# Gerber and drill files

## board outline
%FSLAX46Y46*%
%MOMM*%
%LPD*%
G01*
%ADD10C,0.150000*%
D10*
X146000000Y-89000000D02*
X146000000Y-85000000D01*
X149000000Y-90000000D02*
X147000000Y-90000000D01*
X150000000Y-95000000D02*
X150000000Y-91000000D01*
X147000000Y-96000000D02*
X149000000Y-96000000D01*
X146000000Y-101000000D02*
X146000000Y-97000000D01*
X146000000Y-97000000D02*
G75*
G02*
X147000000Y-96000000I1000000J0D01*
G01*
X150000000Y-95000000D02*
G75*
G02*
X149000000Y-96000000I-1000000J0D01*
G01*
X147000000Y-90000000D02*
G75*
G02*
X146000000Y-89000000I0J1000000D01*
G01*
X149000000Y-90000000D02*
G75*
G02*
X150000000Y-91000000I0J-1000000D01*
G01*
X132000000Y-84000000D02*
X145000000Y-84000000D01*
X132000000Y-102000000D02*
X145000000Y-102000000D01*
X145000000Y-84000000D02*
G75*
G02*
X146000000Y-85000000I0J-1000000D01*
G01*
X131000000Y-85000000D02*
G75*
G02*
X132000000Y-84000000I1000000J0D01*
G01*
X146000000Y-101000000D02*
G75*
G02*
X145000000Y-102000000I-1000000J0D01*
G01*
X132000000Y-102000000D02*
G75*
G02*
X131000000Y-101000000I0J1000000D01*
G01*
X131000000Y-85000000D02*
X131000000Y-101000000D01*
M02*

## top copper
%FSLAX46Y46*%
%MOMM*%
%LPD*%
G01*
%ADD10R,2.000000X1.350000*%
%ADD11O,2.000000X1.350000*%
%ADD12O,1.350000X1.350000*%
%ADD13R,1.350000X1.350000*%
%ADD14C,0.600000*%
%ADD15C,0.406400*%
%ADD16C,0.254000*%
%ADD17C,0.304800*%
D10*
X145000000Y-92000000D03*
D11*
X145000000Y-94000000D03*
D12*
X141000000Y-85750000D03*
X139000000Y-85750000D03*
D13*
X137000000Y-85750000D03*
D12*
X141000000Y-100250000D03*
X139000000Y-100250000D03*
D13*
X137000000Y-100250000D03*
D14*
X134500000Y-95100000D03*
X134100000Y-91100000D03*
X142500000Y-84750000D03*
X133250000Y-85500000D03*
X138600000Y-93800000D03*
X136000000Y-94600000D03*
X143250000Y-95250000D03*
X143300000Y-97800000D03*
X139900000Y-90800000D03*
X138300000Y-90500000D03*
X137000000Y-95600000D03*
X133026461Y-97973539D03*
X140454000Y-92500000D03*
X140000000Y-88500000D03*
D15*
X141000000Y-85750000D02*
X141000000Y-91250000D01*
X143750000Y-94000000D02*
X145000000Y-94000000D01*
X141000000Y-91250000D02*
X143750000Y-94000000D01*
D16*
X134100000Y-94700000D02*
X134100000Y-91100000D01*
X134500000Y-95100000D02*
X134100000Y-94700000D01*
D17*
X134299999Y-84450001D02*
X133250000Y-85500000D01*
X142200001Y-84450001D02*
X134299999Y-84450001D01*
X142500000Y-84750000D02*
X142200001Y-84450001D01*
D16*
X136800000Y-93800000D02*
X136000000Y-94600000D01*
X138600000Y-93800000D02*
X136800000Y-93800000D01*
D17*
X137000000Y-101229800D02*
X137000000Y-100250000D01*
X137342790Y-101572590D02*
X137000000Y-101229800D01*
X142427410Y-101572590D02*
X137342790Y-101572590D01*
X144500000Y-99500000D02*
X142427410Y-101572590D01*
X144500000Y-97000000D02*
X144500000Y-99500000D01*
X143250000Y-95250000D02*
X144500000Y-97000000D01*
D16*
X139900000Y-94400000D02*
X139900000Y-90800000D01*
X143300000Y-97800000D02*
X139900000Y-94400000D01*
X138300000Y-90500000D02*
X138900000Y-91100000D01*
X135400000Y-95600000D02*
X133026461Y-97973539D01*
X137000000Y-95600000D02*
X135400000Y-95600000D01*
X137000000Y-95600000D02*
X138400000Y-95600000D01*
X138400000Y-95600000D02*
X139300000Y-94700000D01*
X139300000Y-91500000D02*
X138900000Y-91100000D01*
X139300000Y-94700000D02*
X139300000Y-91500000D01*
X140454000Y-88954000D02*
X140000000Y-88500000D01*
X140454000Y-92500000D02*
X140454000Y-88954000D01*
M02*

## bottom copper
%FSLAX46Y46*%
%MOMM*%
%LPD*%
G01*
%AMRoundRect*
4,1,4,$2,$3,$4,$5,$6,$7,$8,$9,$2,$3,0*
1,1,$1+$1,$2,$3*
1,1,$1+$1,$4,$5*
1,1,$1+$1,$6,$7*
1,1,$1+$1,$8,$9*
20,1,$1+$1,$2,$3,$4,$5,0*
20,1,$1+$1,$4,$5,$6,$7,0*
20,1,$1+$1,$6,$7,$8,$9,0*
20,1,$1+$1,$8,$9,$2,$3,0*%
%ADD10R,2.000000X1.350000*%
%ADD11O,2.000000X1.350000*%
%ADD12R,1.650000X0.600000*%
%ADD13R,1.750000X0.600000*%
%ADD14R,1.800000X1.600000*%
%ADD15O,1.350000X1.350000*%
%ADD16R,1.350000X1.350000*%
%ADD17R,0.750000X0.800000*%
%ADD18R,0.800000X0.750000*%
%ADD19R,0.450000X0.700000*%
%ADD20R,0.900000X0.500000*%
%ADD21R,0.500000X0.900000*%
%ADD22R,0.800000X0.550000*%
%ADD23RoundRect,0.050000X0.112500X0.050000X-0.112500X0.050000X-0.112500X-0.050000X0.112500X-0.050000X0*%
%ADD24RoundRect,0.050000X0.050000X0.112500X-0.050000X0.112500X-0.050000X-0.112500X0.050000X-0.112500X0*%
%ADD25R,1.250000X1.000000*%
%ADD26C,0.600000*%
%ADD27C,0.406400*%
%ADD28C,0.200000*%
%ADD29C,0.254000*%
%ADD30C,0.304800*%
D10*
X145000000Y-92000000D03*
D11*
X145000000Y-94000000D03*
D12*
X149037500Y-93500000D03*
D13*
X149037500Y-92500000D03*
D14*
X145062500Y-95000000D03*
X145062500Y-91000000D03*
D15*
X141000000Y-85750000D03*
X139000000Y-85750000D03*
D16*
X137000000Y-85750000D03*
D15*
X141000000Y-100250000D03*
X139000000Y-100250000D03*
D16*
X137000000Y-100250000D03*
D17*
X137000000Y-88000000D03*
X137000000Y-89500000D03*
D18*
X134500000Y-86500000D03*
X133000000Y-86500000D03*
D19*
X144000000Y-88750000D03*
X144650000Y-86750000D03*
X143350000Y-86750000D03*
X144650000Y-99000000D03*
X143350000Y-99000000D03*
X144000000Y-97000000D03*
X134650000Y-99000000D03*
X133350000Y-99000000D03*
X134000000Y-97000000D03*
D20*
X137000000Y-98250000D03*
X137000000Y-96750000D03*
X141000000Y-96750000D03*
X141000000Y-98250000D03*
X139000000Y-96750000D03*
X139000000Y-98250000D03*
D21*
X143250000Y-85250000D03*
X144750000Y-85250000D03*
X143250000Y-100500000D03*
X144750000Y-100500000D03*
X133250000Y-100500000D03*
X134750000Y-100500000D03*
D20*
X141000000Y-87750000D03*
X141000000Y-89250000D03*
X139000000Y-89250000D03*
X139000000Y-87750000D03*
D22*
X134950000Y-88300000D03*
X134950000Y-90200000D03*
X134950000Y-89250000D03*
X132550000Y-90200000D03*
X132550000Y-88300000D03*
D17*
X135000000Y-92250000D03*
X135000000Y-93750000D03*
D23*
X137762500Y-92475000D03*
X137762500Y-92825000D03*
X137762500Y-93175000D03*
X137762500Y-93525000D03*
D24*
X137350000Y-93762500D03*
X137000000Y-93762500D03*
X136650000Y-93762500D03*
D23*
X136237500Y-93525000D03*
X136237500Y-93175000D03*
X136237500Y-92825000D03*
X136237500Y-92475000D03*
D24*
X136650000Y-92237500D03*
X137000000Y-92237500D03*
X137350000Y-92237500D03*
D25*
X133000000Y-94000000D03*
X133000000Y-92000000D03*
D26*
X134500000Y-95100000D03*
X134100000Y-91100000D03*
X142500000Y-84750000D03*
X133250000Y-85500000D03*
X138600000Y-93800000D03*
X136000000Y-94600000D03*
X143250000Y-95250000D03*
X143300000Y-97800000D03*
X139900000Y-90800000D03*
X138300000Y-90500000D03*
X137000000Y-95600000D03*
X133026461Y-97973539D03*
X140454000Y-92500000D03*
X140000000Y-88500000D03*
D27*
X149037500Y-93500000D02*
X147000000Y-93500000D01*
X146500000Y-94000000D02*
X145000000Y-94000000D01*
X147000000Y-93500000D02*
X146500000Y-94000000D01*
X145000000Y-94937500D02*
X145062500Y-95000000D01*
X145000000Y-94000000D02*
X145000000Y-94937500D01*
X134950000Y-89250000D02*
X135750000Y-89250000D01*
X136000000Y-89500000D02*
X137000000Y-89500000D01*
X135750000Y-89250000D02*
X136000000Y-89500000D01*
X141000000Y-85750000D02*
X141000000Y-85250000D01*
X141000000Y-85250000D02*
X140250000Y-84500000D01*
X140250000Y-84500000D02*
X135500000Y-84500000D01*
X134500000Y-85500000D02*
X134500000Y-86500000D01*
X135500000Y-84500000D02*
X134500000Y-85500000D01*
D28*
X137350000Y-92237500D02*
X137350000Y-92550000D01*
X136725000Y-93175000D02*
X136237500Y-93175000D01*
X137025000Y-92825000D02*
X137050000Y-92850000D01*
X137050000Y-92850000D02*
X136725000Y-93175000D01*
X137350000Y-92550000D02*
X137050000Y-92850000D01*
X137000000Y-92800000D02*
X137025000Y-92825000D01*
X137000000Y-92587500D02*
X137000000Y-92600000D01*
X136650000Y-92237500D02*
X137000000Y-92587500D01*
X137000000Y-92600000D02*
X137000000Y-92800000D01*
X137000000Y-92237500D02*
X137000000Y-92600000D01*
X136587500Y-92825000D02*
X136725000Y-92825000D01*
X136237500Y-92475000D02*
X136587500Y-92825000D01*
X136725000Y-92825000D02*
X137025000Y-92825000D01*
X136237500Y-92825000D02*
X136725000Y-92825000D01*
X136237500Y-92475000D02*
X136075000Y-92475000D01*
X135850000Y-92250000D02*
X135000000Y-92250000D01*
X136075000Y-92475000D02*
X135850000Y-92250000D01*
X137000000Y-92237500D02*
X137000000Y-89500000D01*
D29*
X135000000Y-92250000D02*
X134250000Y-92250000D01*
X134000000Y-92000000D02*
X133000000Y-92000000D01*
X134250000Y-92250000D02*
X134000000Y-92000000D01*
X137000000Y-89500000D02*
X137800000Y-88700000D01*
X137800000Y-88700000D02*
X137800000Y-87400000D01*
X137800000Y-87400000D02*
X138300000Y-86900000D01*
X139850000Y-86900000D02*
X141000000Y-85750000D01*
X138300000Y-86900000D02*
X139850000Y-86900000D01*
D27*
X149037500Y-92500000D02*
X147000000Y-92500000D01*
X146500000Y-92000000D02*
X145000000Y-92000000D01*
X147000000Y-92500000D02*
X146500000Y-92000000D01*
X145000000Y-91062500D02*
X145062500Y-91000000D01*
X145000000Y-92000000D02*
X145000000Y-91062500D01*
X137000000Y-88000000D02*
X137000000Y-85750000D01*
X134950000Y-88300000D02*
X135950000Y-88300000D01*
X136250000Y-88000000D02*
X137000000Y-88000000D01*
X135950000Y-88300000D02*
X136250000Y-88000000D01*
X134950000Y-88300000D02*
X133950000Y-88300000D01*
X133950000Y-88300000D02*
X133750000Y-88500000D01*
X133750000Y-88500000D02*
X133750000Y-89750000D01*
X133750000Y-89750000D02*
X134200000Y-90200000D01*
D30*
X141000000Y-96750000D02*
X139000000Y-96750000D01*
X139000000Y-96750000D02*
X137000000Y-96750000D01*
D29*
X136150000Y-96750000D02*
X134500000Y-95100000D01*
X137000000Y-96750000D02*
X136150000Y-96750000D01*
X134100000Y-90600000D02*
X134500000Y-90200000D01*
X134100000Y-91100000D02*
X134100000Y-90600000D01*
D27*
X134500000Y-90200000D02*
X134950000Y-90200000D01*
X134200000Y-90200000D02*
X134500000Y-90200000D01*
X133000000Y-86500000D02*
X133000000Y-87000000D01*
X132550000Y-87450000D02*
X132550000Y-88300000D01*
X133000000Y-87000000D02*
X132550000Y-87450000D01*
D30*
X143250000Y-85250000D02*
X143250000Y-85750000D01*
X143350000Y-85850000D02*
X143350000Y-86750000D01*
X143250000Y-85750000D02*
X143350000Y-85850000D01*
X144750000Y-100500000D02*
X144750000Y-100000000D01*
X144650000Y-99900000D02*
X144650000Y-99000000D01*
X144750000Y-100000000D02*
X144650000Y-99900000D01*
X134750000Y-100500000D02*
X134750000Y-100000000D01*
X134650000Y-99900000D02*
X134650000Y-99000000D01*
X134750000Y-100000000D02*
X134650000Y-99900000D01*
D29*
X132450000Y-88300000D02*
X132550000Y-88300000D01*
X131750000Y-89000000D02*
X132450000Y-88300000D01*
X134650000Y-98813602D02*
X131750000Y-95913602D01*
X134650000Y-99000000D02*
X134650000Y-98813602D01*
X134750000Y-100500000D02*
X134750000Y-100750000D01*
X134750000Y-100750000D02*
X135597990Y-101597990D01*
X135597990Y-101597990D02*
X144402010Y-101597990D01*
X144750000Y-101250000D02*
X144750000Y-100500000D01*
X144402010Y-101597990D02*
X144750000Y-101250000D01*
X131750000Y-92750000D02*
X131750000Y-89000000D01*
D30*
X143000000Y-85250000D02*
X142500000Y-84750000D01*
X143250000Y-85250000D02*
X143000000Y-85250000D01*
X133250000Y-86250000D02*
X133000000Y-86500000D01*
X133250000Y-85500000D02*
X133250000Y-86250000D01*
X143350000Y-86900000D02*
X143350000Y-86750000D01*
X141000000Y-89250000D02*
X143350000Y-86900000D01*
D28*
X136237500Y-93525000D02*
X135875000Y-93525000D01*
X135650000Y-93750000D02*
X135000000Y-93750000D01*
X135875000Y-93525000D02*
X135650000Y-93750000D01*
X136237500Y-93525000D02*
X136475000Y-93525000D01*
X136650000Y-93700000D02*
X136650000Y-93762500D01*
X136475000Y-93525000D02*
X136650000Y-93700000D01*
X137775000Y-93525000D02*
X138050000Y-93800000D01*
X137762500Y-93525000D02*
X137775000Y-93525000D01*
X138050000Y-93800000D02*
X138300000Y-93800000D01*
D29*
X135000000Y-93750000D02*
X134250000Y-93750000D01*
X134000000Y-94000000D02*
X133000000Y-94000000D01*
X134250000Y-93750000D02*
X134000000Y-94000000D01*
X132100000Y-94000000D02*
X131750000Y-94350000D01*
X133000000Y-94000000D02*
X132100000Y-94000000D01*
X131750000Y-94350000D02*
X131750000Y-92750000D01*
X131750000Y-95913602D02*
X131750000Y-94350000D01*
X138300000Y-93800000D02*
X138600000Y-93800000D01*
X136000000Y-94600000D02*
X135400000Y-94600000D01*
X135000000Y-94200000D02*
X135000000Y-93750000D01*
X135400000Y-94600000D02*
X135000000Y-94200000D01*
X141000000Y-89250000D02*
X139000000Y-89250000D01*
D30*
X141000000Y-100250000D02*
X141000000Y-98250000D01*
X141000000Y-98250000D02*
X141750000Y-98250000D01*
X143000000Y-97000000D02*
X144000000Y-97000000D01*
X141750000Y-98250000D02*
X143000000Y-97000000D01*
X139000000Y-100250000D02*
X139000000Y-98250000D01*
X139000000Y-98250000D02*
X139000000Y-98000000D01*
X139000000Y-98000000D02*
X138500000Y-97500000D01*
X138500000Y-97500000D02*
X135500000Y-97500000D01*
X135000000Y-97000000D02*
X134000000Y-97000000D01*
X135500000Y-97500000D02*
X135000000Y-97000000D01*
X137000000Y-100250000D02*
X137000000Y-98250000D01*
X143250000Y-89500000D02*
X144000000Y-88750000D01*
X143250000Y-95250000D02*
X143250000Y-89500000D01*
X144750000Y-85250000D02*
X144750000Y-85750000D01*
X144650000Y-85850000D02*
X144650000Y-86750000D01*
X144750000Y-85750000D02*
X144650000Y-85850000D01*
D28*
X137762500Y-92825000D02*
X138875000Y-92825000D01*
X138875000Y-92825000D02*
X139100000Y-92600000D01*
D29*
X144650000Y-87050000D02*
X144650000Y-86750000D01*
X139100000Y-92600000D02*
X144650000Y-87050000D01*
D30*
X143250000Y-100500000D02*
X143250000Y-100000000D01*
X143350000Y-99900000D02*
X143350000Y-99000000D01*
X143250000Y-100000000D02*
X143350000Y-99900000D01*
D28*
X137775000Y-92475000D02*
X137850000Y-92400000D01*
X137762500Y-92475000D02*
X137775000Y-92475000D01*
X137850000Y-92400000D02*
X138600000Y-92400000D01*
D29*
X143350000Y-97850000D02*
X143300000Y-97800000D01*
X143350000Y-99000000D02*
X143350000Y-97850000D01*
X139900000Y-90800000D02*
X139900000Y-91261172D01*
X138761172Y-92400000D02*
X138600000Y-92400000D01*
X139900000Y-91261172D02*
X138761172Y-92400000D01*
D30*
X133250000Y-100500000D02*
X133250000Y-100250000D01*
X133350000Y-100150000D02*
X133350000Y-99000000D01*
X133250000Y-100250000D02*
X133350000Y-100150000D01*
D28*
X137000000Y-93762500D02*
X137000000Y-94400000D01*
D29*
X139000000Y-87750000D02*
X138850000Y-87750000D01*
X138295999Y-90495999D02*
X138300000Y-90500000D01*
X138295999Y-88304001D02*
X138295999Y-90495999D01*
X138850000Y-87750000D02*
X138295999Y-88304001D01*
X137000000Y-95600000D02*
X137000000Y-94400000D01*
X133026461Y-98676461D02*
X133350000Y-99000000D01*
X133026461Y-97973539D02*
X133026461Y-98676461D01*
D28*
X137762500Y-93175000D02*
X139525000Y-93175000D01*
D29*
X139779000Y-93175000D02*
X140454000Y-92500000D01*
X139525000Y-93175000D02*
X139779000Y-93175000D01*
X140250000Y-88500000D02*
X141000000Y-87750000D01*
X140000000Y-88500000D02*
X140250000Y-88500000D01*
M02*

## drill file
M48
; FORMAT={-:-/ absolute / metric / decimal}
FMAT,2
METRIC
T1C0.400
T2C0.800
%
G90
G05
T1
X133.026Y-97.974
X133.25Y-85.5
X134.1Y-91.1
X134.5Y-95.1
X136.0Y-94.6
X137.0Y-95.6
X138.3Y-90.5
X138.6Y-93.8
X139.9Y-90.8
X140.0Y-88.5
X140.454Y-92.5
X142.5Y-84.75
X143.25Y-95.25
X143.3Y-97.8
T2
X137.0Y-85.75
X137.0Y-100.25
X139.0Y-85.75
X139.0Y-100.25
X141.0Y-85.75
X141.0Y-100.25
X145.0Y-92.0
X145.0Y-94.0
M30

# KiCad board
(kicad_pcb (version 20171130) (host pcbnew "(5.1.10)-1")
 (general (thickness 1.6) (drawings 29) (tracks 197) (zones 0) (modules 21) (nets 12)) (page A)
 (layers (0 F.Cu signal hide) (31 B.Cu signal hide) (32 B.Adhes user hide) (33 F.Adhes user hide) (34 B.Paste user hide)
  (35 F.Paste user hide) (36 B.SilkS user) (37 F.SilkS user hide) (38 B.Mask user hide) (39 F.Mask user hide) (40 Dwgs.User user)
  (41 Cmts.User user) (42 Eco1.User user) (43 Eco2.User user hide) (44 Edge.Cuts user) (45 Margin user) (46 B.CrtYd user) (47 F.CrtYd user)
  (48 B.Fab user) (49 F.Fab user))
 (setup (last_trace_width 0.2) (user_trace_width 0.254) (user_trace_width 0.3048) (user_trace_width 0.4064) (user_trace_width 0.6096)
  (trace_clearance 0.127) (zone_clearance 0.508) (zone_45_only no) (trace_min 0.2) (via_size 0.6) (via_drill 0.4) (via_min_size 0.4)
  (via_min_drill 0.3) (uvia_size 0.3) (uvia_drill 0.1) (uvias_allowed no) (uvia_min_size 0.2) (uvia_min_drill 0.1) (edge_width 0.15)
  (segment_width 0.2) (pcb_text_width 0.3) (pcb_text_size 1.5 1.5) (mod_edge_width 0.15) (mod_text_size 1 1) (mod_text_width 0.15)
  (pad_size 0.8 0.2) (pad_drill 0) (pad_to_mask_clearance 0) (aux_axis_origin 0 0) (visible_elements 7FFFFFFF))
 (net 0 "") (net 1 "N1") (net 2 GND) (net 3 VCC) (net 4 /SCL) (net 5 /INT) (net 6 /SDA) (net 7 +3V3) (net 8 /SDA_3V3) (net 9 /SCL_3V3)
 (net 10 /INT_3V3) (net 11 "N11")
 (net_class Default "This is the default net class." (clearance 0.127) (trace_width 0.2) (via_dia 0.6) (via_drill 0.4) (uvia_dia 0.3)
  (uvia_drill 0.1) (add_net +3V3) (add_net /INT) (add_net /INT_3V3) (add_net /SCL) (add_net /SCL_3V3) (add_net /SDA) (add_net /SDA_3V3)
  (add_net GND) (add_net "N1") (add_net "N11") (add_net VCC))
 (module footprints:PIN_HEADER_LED (layer B.Cu) (at 145 92 180)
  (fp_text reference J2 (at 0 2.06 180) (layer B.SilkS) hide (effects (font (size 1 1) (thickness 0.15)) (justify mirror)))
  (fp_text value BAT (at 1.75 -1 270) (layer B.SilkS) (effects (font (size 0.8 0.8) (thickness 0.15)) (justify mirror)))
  (pad 1 thru_hole rect (at 0 0 180) (size 2 1.35) (drill 0.8) (layers *.Cu *.Mask) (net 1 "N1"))
  (pad 2 thru_hole oval (at 0 -2 180) (size 2 1.35) (drill 0.8) (layers *.Cu *.Mask) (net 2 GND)))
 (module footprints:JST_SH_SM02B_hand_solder (layer B.Cu) (at 147 93 90)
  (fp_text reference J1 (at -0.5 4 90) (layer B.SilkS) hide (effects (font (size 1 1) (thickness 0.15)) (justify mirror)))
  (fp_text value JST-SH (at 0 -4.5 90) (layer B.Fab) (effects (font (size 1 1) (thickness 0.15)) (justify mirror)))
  (pad 1 smd rect (at -0.5 2.0375 90) (size 0.6 1.65) (layers B.Cu B.Paste B.Mask) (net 2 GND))
  (pad 2 smd rect (at 0.5 2.0375 90) (size 0.6 1.75) (layers B.Cu B.Paste B.Mask) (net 1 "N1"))
  (pad 1 smd rect (at -2 -1.9375 90) (size 1.6 1.8) (layers B.Cu B.Paste B.Mask) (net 2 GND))
  (pad 2 smd rect (at 2 -1.9375 90) (size 1.6 1.8) (layers B.Cu B.Paste B.Mask) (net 1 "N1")))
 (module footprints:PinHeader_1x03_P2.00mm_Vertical (layer B.Cu) (at 137 85.75 270)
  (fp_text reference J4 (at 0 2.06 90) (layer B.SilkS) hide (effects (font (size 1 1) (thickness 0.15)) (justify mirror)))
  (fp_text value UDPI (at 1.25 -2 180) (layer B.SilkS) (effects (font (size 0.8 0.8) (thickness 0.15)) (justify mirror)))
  (pad 3 thru_hole oval (at 0 -4 270) (size 1.35 1.35) (drill 0.8) (layers *.Cu *.Mask) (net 2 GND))
  (pad 2 thru_hole oval (at 0 -2 270) (size 1.35 1.35) (drill 0.8) (layers *.Cu *.Mask))
  (pad 1 thru_hole rect (at 0 0 270) (size 1.35 1.35) (drill 0.8) (layers *.Cu *.Mask) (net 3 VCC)))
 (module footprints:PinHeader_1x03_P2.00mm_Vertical (layer B.Cu) (at 137 100.25 270)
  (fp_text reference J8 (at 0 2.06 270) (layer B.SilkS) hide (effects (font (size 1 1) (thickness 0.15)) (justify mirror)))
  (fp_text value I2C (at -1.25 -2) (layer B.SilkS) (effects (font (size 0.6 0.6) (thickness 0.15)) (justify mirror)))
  (pad 3 thru_hole oval (at 0 -4 270) (size 1.35 1.35) (drill 0.8) (layers *.Cu *.Mask) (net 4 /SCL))
  (pad 2 thru_hole oval (at 0 -2 270) (size 1.35 1.35) (drill 0.8) (layers *.Cu *.Mask) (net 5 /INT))
  (pad 1 thru_hole rect (at 0 0 270) (size 1.35 1.35) (drill 0.8) (layers *.Cu *.Mask) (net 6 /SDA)))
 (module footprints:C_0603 (layer B.Cu) (at 137 88.75 270)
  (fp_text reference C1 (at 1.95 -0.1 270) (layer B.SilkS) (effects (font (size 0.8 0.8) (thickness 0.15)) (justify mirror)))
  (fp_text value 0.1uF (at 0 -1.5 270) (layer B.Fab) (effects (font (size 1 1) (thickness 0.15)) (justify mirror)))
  (pad 1 smd rect (at -0.75 0 270) (size 0.8 0.75) (layers B.Cu B.Paste B.Mask) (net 3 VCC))
  (pad 2 smd rect (at 0.75 0 270) (size 0.8 0.75) (layers B.Cu B.Paste B.Mask) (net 2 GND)))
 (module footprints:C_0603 (layer B.Cu) (at 133.75 86.5)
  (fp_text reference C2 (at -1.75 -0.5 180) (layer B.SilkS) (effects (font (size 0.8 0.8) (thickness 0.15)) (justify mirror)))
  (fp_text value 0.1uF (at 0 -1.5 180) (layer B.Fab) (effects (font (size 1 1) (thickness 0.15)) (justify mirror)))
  (pad 2 smd rect (at 0.75 0) (size 0.8 0.75) (layers B.Cu B.Paste B.Mask) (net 2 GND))
  (pad 1 smd rect (at -0.75 0) (size 0.8 0.75) (layers B.Cu B.Paste B.Mask) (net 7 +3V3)))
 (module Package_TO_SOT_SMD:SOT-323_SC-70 (layer B.Cu) (at 144 87.75 270)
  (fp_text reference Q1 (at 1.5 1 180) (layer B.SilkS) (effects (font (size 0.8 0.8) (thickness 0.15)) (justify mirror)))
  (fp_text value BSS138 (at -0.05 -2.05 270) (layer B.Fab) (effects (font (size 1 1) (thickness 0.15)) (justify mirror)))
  (pad 3 smd rect (at 1 0) (size 0.45 0.7) (layers B.Cu B.Paste B.Mask) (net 6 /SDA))
  (pad 2 smd rect (at -1 -0.65) (size 0.45 0.7) (layers B.Cu B.Paste B.Mask) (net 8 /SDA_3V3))
  (pad 1 smd rect (at -1 0.65) (size 0.45 0.7) (layers B.Cu B.Paste B.Mask) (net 7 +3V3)))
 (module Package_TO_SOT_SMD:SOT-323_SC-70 (layer B.Cu) (at 144 98 90)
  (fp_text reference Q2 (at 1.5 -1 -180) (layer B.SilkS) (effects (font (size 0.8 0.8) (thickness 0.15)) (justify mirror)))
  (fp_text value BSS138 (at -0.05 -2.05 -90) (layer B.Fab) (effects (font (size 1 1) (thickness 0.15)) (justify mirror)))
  (pad 1 smd rect (at -1 0.65 180) (size 0.45 0.7) (layers B.Cu B.Paste B.Mask) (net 7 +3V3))
  (pad 2 smd rect (at -1 -0.65 180) (size 0.45 0.7) (layers B.Cu B.Paste B.Mask) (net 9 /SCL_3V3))
  (pad 3 smd rect (at 1 0 180) (size 0.45 0.7) (layers B.Cu B.Paste B.Mask) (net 4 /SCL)))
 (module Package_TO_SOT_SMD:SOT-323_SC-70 (layer B.Cu) (at 134 98 90)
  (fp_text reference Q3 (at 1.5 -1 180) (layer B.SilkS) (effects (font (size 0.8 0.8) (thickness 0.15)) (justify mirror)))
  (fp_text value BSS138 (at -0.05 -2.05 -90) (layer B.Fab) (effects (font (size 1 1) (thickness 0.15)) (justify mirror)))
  (pad 1 smd rect (at -1 0.65 180) (size 0.45 0.7) (layers B.Cu B.Paste B.Mask) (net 7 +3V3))
  (pad 2 smd rect (at -1 -0.65 180) (size 0.45 0.7) (layers B.Cu B.Paste B.Mask) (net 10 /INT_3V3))
  (pad 3 smd rect (at 1 0 180) (size 0.45 0.7) (layers B.Cu B.Paste B.Mask) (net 5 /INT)))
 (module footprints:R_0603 (layer B.Cu) (at 137 97.5 270)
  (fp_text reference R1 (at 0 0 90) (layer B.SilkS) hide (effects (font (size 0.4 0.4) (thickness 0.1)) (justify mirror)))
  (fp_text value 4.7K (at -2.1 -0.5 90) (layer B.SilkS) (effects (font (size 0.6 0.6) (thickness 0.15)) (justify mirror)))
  (pad 2 smd rect (at 0.75 0 270) (size 0.5 0.9) (layers B.Cu B.Paste B.Mask) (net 6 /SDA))
  (pad 1 smd rect (at -0.75 0 270) (size 0.5 0.9) (layers B.Cu B.Paste B.Mask) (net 3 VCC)))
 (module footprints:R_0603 (layer B.Cu) (at 141 97.5 270)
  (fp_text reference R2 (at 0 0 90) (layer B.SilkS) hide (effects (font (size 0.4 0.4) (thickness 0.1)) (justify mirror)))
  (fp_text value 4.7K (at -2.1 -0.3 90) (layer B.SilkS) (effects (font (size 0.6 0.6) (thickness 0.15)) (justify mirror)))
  (pad 1 smd rect (at -0.75 0 270) (size 0.5 0.9) (layers B.Cu B.Paste B.Mask) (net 3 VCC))
  (pad 2 smd rect (at 0.75 0 270) (size 0.5 0.9) (layers B.Cu B.Paste B.Mask) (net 4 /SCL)))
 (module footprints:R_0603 (layer B.Cu) (at 139 97.5 270)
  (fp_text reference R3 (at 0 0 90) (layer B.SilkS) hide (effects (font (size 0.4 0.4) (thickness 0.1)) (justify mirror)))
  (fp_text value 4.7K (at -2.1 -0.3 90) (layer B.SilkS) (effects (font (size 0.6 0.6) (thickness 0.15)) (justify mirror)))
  (pad 1 smd rect (at -0.75 0 270) (size 0.5 0.9) (layers B.Cu B.Paste B.Mask) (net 3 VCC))
  (pad 2 smd rect (at 0.75 0 270) (size 0.5 0.9) (layers B.Cu B.Paste B.Mask) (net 5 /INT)))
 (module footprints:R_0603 (layer B.Cu) (at 144 85.25)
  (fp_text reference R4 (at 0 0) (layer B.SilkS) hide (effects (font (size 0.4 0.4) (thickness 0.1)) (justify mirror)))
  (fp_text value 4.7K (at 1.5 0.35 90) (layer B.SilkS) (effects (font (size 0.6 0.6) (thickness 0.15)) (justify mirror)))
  (pad 1 smd rect (at -0.75 0) (size 0.5 0.9) (layers B.Cu B.Paste B.Mask) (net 7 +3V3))
  (pad 2 smd rect (at 0.75 0) (size 0.5 0.9) (layers B.Cu B.Paste B.Mask) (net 8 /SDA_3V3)))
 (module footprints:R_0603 (layer B.Cu) (at 144 100.5 180)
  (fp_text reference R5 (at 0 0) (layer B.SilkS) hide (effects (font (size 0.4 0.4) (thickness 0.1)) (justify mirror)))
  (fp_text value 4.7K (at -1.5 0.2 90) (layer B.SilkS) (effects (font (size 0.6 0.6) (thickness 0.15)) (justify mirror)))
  (pad 2 smd rect (at 0.75 0 180) (size 0.5 0.9) (layers B.Cu B.Paste B.Mask) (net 9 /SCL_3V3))
  (pad 1 smd rect (at -0.75 0 180) (size 0.5 0.9) (layers B.Cu B.Paste B.Mask) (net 7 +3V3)))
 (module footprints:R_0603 (layer B.Cu) (at 134 100.5 180)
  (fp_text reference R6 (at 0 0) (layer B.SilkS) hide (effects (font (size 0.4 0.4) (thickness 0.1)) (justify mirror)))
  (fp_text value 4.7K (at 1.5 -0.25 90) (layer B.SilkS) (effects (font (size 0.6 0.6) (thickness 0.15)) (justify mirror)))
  (pad 2 smd rect (at 0.75 0 180) (size 0.5 0.9) (layers B.Cu B.Paste B.Mask) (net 10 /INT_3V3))
  (pad 1 smd rect (at -0.75 0 180) (size 0.5 0.9) (layers B.Cu B.Paste B.Mask) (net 7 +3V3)))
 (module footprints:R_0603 (layer B.Cu) (at 141 88.5 90)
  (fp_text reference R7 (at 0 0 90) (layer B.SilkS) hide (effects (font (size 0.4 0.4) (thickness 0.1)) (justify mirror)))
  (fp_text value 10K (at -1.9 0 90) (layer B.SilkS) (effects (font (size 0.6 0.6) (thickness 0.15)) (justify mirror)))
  (pad 2 smd rect (at 0.75 0 90) (size 0.5 0.9) (layers B.Cu B.Paste B.Mask) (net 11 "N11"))
  (pad 1 smd rect (at -0.75 0 90) (size 0.5 0.9) (layers B.Cu B.Paste B.Mask) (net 7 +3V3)))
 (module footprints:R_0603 (layer B.Cu) (at 139 88.5 90)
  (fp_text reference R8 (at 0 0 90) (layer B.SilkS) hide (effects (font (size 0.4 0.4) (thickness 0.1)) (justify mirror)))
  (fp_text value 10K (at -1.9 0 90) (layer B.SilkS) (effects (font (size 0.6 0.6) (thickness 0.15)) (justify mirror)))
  (pad 1 smd rect (at -0.75 0 90) (size 0.5 0.9) (layers B.Cu B.Paste B.Mask) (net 7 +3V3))
  (pad 2 smd rect (at 0.75 0 90) (size 0.5 0.9) (layers B.Cu B.Paste B.Mask) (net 10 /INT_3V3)))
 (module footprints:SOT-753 (layer B.Cu) (at 133.75 89.25 270) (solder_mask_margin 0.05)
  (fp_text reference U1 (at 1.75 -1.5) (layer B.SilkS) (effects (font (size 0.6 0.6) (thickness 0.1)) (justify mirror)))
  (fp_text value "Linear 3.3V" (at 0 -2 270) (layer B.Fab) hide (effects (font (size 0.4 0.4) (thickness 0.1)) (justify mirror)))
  (pad 1 smd rect (at -0.95 -1.2 270) (size 0.55 0.8) (layers B.Cu B.Paste B.Mask) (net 3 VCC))
  (pad 3 smd rect (at 0.95 -1.2 270) (size 0.55 0.8) (layers B.Cu B.Paste B.Mask) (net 3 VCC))
  (pad 2 smd rect (at 0 -1.2 270) (size 0.55 0.8) (layers B.Cu B.Paste B.Mask) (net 2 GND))
  (pad 4 smd rect (at 0.95 1.2 270) (size 0.55 0.8) (layers B.Cu B.Paste B.Mask))
  (pad 5 smd rect (at -0.95 1.2 270) (size 0.55 0.8) (layers B.Cu B.Paste B.Mask) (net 7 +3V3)))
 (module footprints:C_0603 (layer B.Cu) (at 135 93 90)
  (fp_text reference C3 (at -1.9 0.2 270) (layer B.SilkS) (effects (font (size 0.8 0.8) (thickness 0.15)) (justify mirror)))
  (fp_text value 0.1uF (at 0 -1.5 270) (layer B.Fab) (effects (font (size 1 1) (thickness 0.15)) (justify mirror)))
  (pad 2 smd rect (at 0.75 0 90) (size 0.8 0.75) (layers B.Cu B.Paste B.Mask) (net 2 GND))
  (pad 1 smd rect (at -0.75 0 90) (size 0.8 0.75) (layers B.Cu B.Paste B.Mask) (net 7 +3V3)))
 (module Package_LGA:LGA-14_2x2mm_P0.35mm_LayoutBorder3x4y (layer B.Cu) (at 137 93 180) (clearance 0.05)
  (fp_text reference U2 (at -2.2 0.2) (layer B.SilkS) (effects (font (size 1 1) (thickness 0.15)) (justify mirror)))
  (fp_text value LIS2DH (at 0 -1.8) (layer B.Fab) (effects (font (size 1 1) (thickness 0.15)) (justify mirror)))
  (pad 1 smd roundrect (at -0.7625 0.525 180) (size 0.325 0.2) (layers B.Cu B.Paste B.Mask) (roundrect_rratio 0.25) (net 9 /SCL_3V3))
  (pad 2 smd roundrect (at -0.7625 0.175 180) (size 0.325 0.2) (layers B.Cu B.Paste B.Mask) (roundrect_rratio 0.25) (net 8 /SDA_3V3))
  (pad 3 smd roundrect (at -0.7625 -0.175 180) (size 0.325 0.2) (layers B.Cu B.Paste B.Mask) (roundrect_rratio 0.25) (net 11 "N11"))
  (pad 4 smd roundrect (at -0.7625 -0.525 180) (size 0.325 0.2) (layers B.Cu B.Paste B.Mask) (roundrect_rratio 0.25) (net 7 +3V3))
  (pad 5 smd roundrect (at -0.35 -0.7625 180) (size 0.2 0.325) (layers B.Cu B.Paste B.Mask) (roundrect_rratio 0.25))
  (pad 6 smd roundrect (at 0 -0.7625 180) (size 0.2 0.325) (layers B.Cu B.Paste B.Mask) (roundrect_rratio 0.25) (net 10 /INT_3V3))
  (pad 7 smd roundrect (at 0.35 -0.7625 180) (size 0.2 0.325) (layers B.Cu B.Paste B.Mask) (roundrect_rratio 0.25) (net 7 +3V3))
  (pad 8 smd roundrect (at 0.7625 -0.525 180) (size 0.325 0.2) (layers B.Cu B.Paste B.Mask) (roundrect_rratio 0.25) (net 7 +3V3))
  (pad 9 smd roundrect (at 0.7625 -0.175 180) (size 0.325 0.2) (layers B.Cu B.Paste B.Mask) (roundrect_rratio 0.25) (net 2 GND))
  (pad 10 smd roundrect (at 0.7625 0.175 180) (size 0.325 0.2) (layers B.Cu B.Paste B.Mask) (roundrect_rratio 0.25) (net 2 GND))
  (pad 11 smd roundrect (at 0.7625 0.525 180) (size 0.325 0.2) (layers B.Cu B.Paste B.Mask) (roundrect_rratio 0.25) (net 2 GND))
  (pad 12 smd roundrect (at 0.35 0.7625 180) (size 0.2 0.325) (layers B.Cu B.Paste B.Mask) (roundrect_rratio 0.25) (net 2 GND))
  (pad 13 smd roundrect (at 0 0.7625 180) (size 0.2 0.325) (layers B.Cu B.Paste B.Mask) (roundrect_rratio 0.25) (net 2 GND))
  (pad 14 smd roundrect (at -0.35 0.7625 180) (size 0.2 0.325) (layers B.Cu B.Paste B.Mask) (roundrect_rratio 0.25) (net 2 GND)))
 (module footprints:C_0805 (layer B.Cu) (at 133 93 90)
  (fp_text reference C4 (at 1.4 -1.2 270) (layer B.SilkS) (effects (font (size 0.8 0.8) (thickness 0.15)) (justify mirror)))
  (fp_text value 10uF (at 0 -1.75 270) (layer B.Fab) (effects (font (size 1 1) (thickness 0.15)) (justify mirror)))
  (pad 1 smd rect (at -1 0 90) (size 1 1.25) (layers B.Cu B.Paste B.Mask) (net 7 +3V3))
  (pad 2 smd rect (at 1 0 90) (size 1 1.25) (layers B.Cu B.Paste B.Mask) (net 2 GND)))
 (gr_line (start 146 89) (end 146 85) (layer Edge.Cuts) (width 0.15))
 (gr_line (start 149 90) (end 147 90) (layer Edge.Cuts) (width 0.15))
 (gr_line (start 150 95) (end 150 91) (layer Edge.Cuts) (width 0.15))
 (gr_line (start 147 96) (end 149 96) (layer Edge.Cuts) (width 0.15))
 (gr_line (start 146 101) (end 146 97) (layer Edge.Cuts) (width 0.15))
 (gr_arc (start 147 97) (end 147 96) (angle -90) (layer Edge.Cuts) (width 0.15))
 (gr_arc (start 149 95) (end 149 96) (angle -90) (layer Edge.Cuts) (width 0.15))
 (gr_arc (start 147 89) (end 146 89) (angle -90) (layer Edge.Cuts) (width 0.15))
 (gr_arc (start 149 91) (end 150 91) (angle -90) (layer Edge.Cuts) (width 0.15))
 (gr_line (start 132 84) (end 145 84) (layer Edge.Cuts) (width 0.15))
 (gr_line (start 132 102) (end 145 102) (layer Edge.Cuts) (width 0.15))
 (gr_arc (start 145 85) (end 145 84) (angle 90) (layer Edge.Cuts) (width 0.15))
 (gr_arc (start 132 85) (end 131 85) (angle 90) (layer Edge.Cuts) (width 0.15))
 (gr_arc (start 145 101) (end 146 101) (angle 90) (layer Edge.Cuts) (width 0.15))
 (gr_arc (start 132 101) (end 132 102) (angle 90) (layer Edge.Cuts) (width 0.15))
 (gr_line (start 131 85) (end 131 101) (angle 90) (layer Edge.Cuts) (width 0.15))
 (segment (start 149.0375 93.5) (end 147 93.5) (width 0.4064) (layer B.Cu) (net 2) (status 10))
 (segment (start 146.5 94) (end 145 94) (width 0.4064) (layer B.Cu) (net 2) (status 20))
 (segment (start 147 93.5) (end 146.5 94) (width 0.4064) (layer B.Cu) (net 2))
 (segment (start 145 94.9375) (end 145.0625 95) (width 0.4064) (layer B.Cu) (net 2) (status 30))
 (segment (start 145 94) (end 145 94.9375) (width 0.4064) (layer B.Cu) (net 2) (status 30))
 (segment (start 134.95 89.25) (end 135.75 89.25) (width 0.4064) (layer B.Cu) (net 2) (status 10))
 (segment (start 136 89.5) (end 137 89.5) (width 0.4064) (layer B.Cu) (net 2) (status 20))
 (segment (start 135.75 89.25) (end 136 89.5) (width 0.4064) (layer B.Cu) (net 2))
 (segment (start 141 85.75) (end 141 85.25) (width 0.4064) (layer B.Cu) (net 2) (status 30))
 (segment (start 141 85.25) (end 140.25 84.5) (width 0.4064) (layer B.Cu) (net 2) (status 10))
 (segment (start 140.25 84.5) (end 135.5 84.5) (width 0.4064) (layer B.Cu) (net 2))
 (segment (start 134.5 85.5) (end 134.5 86.5) (width 0.4064) (layer B.Cu) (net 2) (status 20))
 (segment (start 135.5 84.5) (end 134.5 85.5) (width 0.4064) (layer B.Cu) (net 2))
 (segment (start 141 85.75) (end 141 91.25) (width 0.4064) (layer F.Cu) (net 2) (status 10))
 (segment (start 143.75 94) (end 145 94) (width 0.4064) (layer F.Cu) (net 2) (status 20))
 (segment (start 141 91.25) (end 143.75 94) (width 0.4064) (layer F.Cu) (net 2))
 (segment (start 137.35 92.2375) (end 137.35 92.55) (width 0.2) (layer B.Cu) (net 2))
 (segment (start 136.725 93.175) (end 136.2375 93.175) (width 0.2) (layer B.Cu) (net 2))
 (segment (start 137.025 92.825) (end 137.05 92.85) (width 0.2) (layer B.Cu) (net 2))
 (segment (start 137.05 92.85) (end 136.725 93.175) (width 0.2) (layer B.Cu) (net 2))
 (segment (start 137.35 92.55) (end 137.05 92.85) (width 0.2) (layer B.Cu) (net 2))
 (segment (start 137 92.8) (end 137.025 92.825) (width 0.2) (layer B.Cu) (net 2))
 (segment (start 137 92.5875) (end 137 92.6) (width 0.2) (layer B.Cu) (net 2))
 (segment (start 136.65 92.2375) (end 137 92.5875) (width 0.2) (layer B.Cu) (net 2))
 (segment (start 137 92.6) (end 137 92.8) (width 0.2) (layer B.Cu) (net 2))
 (segment (start 137 92.2375) (end 137 92.6) (width 0.2) (layer B.Cu) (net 2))
 (segment (start 136.5875 92.825) (end 136.725 92.825) (width 0.2) (layer B.Cu) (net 2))
 (segment (start 136.2375 92.475) (end 136.5875 92.825) (width 0.2) (layer B.Cu) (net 2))
 (segment (start 136.725 92.825) (end 137.025 92.825) (width 0.2) (layer B.Cu) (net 2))
 (segment (start 136.2375 92.825) (end 136.725 92.825) (width 0.2) (layer B.Cu) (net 2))
 (segment (start 136.2375 92.475) (end 136.075 92.475) (width 0.2) (layer B.Cu) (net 2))
 (segment (start 135.85 92.25) (end 135 92.25) (width 0.2) (layer B.Cu) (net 2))
 (segment (start 136.075 92.475) (end 135.85 92.25) (width 0.2) (layer B.Cu) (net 2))
 (segment (start 137 92.2375) (end 137 89.5) (width 0.2) (layer B.Cu) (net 2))
 (segment (start 135 92.25) (end 134.25 92.25) (width 0.254) (layer B.Cu) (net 2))
 (segment (start 134 92) (end 133 92) (width 0.254) (layer B.Cu) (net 2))
 (segment (start 134.25 92.25) (end 134 92) (width 0.254) (layer B.Cu) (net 2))
 (segment (start 137 89.5) (end 137.8 88.7) (width 0.254) (layer B.Cu) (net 2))
 (segment (start 137.8 88.7) (end 137.8 87.4) (width 0.254) (layer B.Cu) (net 2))
 (segment (start 137.8 87.4) (end 138.3 86.9) (width 0.254) (layer B.Cu) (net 2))
 (segment (start 139.85 86.9) (end 141 85.75) (width 0.254) (layer B.Cu) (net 2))
 (segment (start 138.3 86.9) (end 139.85 86.9) (width 0.254) (layer B.Cu) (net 2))
 (segment (start 149.0375 92.5) (end 147 92.5) (width 0.4064) (layer B.Cu) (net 1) (status 10))
 (segment (start 146.5 92) (end 145 92) (width 0.4064) (layer B.Cu) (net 1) (status 20))
 (segment (start 147 92.5) (end 146.5 92) (width 0.4064) (layer B.Cu) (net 1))
 (segment (start 145 91.0625) (end 145.0625 91) (width 0.4064) (layer B.Cu) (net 1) (status 30))
 (segment (start 145 92) (end 145 91.0625) (width 0.4064) (layer B.Cu) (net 1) (status 30))
 (segment (start 137 88) (end 137 85.75) (width 0.4064) (layer B.Cu) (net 3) (status 30))
 (segment (start 134.95 88.3) (end 135.95 88.3) (width 0.4064) (layer B.Cu) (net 3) (status 10))
 (segment (start 136.25 88) (end 137 88) (width 0.4064) (layer B.Cu) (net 3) (status 20))
 (segment (start 135.95 88.3) (end 136.25 88) (width 0.4064) (layer B.Cu) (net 3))
 (segment (start 134.95 88.3) (end 133.95 88.3) (width 0.4064) (layer B.Cu) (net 3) (status 10))
 (segment (start 133.95 88.3) (end 133.75 88.5) (width 0.4064) (layer B.Cu) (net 3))
 (segment (start 133.75 88.5) (end 133.75 89.75) (width 0.4064) (layer B.Cu) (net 3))
 (segment (start 133.75 89.75) (end 134.2 90.2) (width 0.4064) (layer B.Cu) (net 3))
 (segment (start 141 96.75) (end 139 96.75) (width 0.3048) (layer B.Cu) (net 3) (status 30))
 (segment (start 139 96.75) (end 137 96.75) (width 0.3048) (layer B.Cu) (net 3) (status 30))
 (via (at 134.5 95.1) (size 0.6) (drill 0.4) (layers F.Cu B.Cu) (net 3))
 (segment (start 136.15 96.75) (end 134.5 95.1) (width 0.254) (layer B.Cu) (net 3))
 (segment (start 137 96.75) (end 136.15 96.75) (width 0.254) (layer B.Cu) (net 3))
 (via (at 134.1 91.1) (size 0.6) (drill 0.4) (layers F.Cu B.Cu) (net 3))
 (segment (start 134.1 94.7) (end 134.1 91.1) (width 0.254) (layer F.Cu) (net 3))
 (segment (start 134.5 95.1) (end 134.1 94.7) (width 0.254) (layer F.Cu) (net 3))
 (segment (start 134.1 90.6) (end 134.5 90.2) (width 0.254) (layer B.Cu) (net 3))
 (segment (start 134.1 91.1) (end 134.1 90.6) (width 0.254) (layer B.Cu) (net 3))
 (segment (start 134.5 90.2) (end 134.95 90.2) (width 0.4064) (layer B.Cu) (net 3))
 (segment (start 134.2 90.2) (end 134.5 90.2) (width 0.4064) (layer B.Cu) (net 3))
 (segment (start 133 86.5) (end 133 87) (width 0.4064) (layer B.Cu) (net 7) (status 10))
 (segment (start 132.55 87.45) (end 132.55 88.3) (width 0.4064) (layer B.Cu) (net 7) (status 20))
 (segment (start 133 87) (end 132.55 87.45) (width 0.4064) (layer B.Cu) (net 7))
 (segment (start 143.25 85.25) (end 143.25 85.75) (width 0.3048) (layer B.Cu) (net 7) (status 10))
 (segment (start 143.35 85.85) (end 143.35 86.75) (width 0.3048) (layer B.Cu) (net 7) (status 20))
 (segment (start 143.25 85.75) (end 143.35 85.85) (width 0.3048) (layer B.Cu) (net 7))
 (segment (start 144.75 100.5) (end 144.75 100) (width 0.3048) (layer B.Cu) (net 7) (status 10))
 (segment (start 144.65 99.9) (end 144.65 99) (width 0.3048) (layer B.Cu) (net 7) (status 20))
 (segment (start 144.75 100) (end 144.65 99.9) (width 0.3048) (layer B.Cu) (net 7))
 (segment (start 134.75 100.5) (end 134.75 100) (width 0.3048) (layer B.Cu) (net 7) (status 10))
 (segment (start 134.65 99.9) (end 134.65 99) (width 0.3048) (layer B.Cu) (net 7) (status 20))
 (segment (start 134.75 100) (end 134.65 99.9) (width 0.3048) (layer B.Cu) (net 7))
 (segment (start 132.45 88.3) (end 132.55 88.3) (width 0.254) (layer B.Cu) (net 7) (status 30))
 (segment (start 131.75 89) (end 132.45 88.3) (width 0.254) (layer B.Cu) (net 7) (status 20))
 (segment (start 134.65 98.813602) (end 131.75 95.913602) (width 0.254) (layer B.Cu) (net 7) (status 10))
 (segment (start 134.65 99) (end 134.65 98.813602) (width 0.254) (layer B.Cu) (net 7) (status 30))
 (segment (start 134.75 100.5) (end 134.75 100.75) (width 0.254) (layer B.Cu) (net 7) (status 30))
 (segment (start 134.75 100.75) (end 135.59799 101.59799) (width 0.254) (layer B.Cu) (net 7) (status 10))
 (segment (start 135.59799 101.59799) (end 144.40201 101.59799) (width 0.254) (layer B.Cu) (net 7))
 (segment (start 144.75 101.25) (end 144.75 100.5) (width 0.254) (layer B.Cu) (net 7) (status 20))
 (segment (start 144.40201 101.59799) (end 144.75 101.25) (width 0.254) (layer B.Cu) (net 7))
 (segment (start 131.75 92.75) (end 131.75 89) (width 0.254) (layer B.Cu) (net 7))
 (via (at 142.5 84.75) (size 0.6) (drill 0.4) (layers F.Cu B.Cu) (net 7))
 (segment (start 143 85.25) (end 142.5 84.75) (width 0.3048) (layer B.Cu) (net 7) (status 10))
 (segment (start 143.25 85.25) (end 143 85.25) (width 0.3048) (layer B.Cu) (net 7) (status 30))
 (via (at 133.25 85.5) (size 0.6) (drill 0.4) (layers F.Cu B.Cu) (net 7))
 (segment (start 134.299999 84.450001) (end 133.25 85.5) (width 0.3048) (layer F.Cu) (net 7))
 (segment (start 142.200001 84.450001) (end 134.299999 84.450001) (width 0.3048) (layer F.Cu) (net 7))
 (segment (start 142.5 84.75) (end 142.200001 84.450001) (width 0.3048) (layer F.Cu) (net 7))
 (segment (start 133.25 86.25) (end 133 86.5) (width 0.3048) (layer B.Cu) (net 7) (status 30))
 (segment (start 133.25 85.5) (end 133.25 86.25) (width 0.3048) (layer B.Cu) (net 7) (status 20))
 (segment (start 143.35 86.9) (end 143.35 86.75) (width 0.3048) (layer B.Cu) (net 7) (status 30))
 (segment (start 141 89.25) (end 143.35 86.9) (width 0.3048) (layer B.Cu) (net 7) (status 30))
 (segment (start 136.2375 93.525) (end 135.875 93.525) (width 0.2) (layer B.Cu) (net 7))
 (segment (start 135.65 93.75) (end 135 93.75) (width 0.2) (layer B.Cu) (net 7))
 (segment (start 135.875 93.525) (end 135.65 93.75) (width 0.2) (layer B.Cu) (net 7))
 (segment (start 136.2375 93.525) (end 136.475 93.525) (width 0.2) (layer B.Cu) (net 7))
 (segment (start 136.65 93.7) (end 136.65 93.7625) (width 0.2) (layer B.Cu) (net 7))
 (segment (start 136.475 93.525) (end 136.65 93.7) (width 0.2) (layer B.Cu) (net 7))
 (segment (start 137.775 93.525) (end 138.05 93.8) (width 0.2) (layer B.Cu) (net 7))
 (segment (start 137.7625 93.525) (end 137.775 93.525) (width 0.2) (layer B.Cu) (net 7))
 (segment (start 138.05 93.8) (end 138.3 93.8) (width 0.2) (layer B.Cu) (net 7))
 (segment (start 135 93.75) (end 134.25 93.75) (width 0.254) (layer B.Cu) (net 7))
 (segment (start 134 94) (end 133 94) (width 0.254) (layer B.Cu) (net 7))
 (segment (start 134.25 93.75) (end 134 94) (width 0.254) (layer B.Cu) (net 7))
 (segment (start 132.1 94) (end 131.75 94.35) (width 0.254) (layer B.Cu) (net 7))
 (segment (start 133 94) (end 132.1 94) (width 0.254) (layer B.Cu) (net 7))
 (segment (start 131.75 94.35) (end 131.75 92.75) (width 0.254) (layer B.Cu) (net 7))
 (segment (start 131.75 95.913602) (end 131.75 94.35) (width 0.254) (layer B.Cu) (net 7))
 (via (at 138.6 93.8) (size 0.6) (drill 0.4) (layers F.Cu B.Cu) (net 7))
 (segment (start 138.3 93.8) (end 138.6 93.8) (width 0.254) (layer B.Cu) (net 7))
 (via (at 136 94.6) (size 0.6) (drill 0.4) (layers F.Cu B.Cu) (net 7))
 (segment (start 136.8 93.8) (end 136 94.6) (width 0.254) (layer F.Cu) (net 7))
 (segment (start 138.6 93.8) (end 136.8 93.8) (width 0.254) (layer F.Cu) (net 7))
 (segment (start 136 94.6) (end 135.4 94.6) (width 0.254) (layer B.Cu) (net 7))
 (segment (start 135 94.2) (end 135 93.75) (width 0.254) (layer B.Cu) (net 7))
 (segment (start 135.4 94.6) (end 135 94.2) (width 0.254) (layer B.Cu) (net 7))
 (segment (start 141 89.25) (end 139 89.25) (width 0.254) (layer B.Cu) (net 7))
 (segment (start 141 100.25) (end 141 98.25) (width 0.3048) (layer B.Cu) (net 4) (status 30))
 (segment (start 141 98.25) (end 141.75 98.25) (width 0.3048) (layer B.Cu) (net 4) (status 10))
 (segment (start 143 97) (end 144 97) (width 0.3048) (layer B.Cu) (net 4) (status 20))
 (segment (start 141.75 98.25) (end 143 97) (width 0.3048) (layer B.Cu) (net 4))
 (segment (start 139 100.25) (end 139 98.25) (width 0.3048) (layer B.Cu) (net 5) (status 30))
 (segment (start 139 98.25) (end 139 98) (width 0.3048) (layer B.Cu) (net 5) (status 30))
 (segment (start 139 98) (end 138.5 97.5) (width 0.3048) (layer B.Cu) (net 5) (status 10))
 (segment (start 138.5 97.5) (end 135.5 97.5) (width 0.3048) (layer B.Cu) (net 5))
 (segment (start 135 97) (end 134 97) (width 0.3048) (layer B.Cu) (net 5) (status 20))
 (segment (start 135.5 97.5) (end 135 97) (width 0.3048) (layer B.Cu) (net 5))
 (segment (start 137 100.25) (end 137 98.25) (width 0.3048) (layer B.Cu) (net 6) (status 30))
 (segment (start 143.25 89.5) (end 144 88.75) (width 0.3048) (layer B.Cu) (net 6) (status 20))
 (segment (start 143.25 95.25) (end 143.25 89.5) (width 0.3048) (layer B.Cu) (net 6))
 (segment (start 137 101.2298) (end 137 100.25) (width 0.3048) (layer F.Cu) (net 6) (status 20))
 (segment (start 137.34279 101.57259) (end 137 101.2298) (width 0.3048) (layer F.Cu) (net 6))
 (segment (start 142.42741 101.57259) (end 137.34279 101.57259) (width 0.3048) (layer F.Cu) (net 6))
 (segment (start 144.5 99.5) (end 142.42741 101.57259) (width 0.3048) (layer F.Cu) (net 6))
 (segment (start 144.5 97) (end 144.5 99.5) (width 0.3048) (layer F.Cu) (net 6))
 (segment (start 143.25 95.25) (end 144.5 97) (width 0.3048) (layer F.Cu) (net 6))
 (via (at 143.25 95.25) (size 0.6) (drill 0.4) (layers F.Cu B.Cu) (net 6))
 (segment (start 144.75 85.25) (end 144.75 85.75) (width 0.3048) (layer B.Cu) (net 8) (status 10))
 (segment (start 144.65 85.85) (end 144.65 86.75) (width 0.3048) (layer B.Cu) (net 8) (status 20))
 (segment (start 144.75 85.75) (end 144.65 85.85) (width 0.3048) (layer B.Cu) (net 8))
 (segment (start 137.7625 92.825) (end 138.875 92.825) (width 0.2) (layer B.Cu) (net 8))
 (segment (start 138.875 92.825) (end 139.1 92.6) (width 0.2) (layer B.Cu) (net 8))
 (segment (start 144.65 87.05) (end 144.65 86.75) (width 0.254) (layer B.Cu) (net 8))
 (segment (start 139.1 92.6) (end 144.65 87.05) (width 0.254) (layer B.Cu) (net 8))
 (segment (start 143.25 100.5) (end 143.25 100) (width 0.3048) (layer B.Cu) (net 9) (status 10))
 (segment (start 143.35 99.9) (end 143.35 99) (width 0.3048) (layer B.Cu) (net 9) (status 20))
 (segment (start 143.25 100) (end 143.35 99.9) (width 0.3048) (layer B.Cu) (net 9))
 (segment (start 137.775 92.475) (end 137.85 92.4) (width 0.2) (layer B.Cu) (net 9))
 (segment (start 137.7625 92.475) (end 137.775 92.475) (width 0.2) (layer B.Cu) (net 9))
 (segment (start 137.85 92.4) (end 138.6 92.4) (width 0.2) (layer B.Cu) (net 9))
 (via (at 143.3 97.8) (size 0.6) (drill 0.4) (layers F.Cu B.Cu) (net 9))
 (segment (start 143.35 97.85) (end 143.3 97.8) (width 0.254) (layer B.Cu) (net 9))
 (segment (start 143.35 99) (end 143.35 97.85) (width 0.254) (layer B.Cu) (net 9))
 (segment (start 139.9 94.4) (end 139.9 90.8) (width 0.254) (layer F.Cu) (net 9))
 (via (at 139.9 90.8) (size 0.6) (drill 0.4) (layers F.Cu B.Cu) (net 9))
 (segment (start 143.3 97.8) (end 139.9 94.4) (width 0.254) (layer F.Cu) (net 9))
 (segment (start 139.9 90.8) (end 139.9 91.261172) (width 0.254) (layer B.Cu) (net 9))
 (segment (start 138.761172 92.4) (end 138.6 92.4) (width 0.254) (layer B.Cu) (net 9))
 (segment (start 139.9 91.261172) (end 138.761172 92.4) (width 0.254) (layer B.Cu) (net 9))
 (segment (start 133.25 100.5) (end 133.25 100.25) (width 0.3048) (layer B.Cu) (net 10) (status 30))
 (segment (start 133.35 100.15) (end 133.35 99) (width 0.3048) (layer B.Cu) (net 10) (status 30))
 (segment (start 133.25 100.25) (end 133.35 100.15) (width 0.3048) (layer B.Cu) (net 10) (status 30))
 (segment (start 137 93.7625) (end 137 94.4) (width 0.2) (layer B.Cu) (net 10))
 (segment (start 139 87.75) (end 138.85 87.75) (width 0.254) (layer B.Cu) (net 10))
 (via (at 138.3 90.5) (size 0.6) (drill 0.4) (layers F.Cu B.Cu) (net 10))
 (segment (start 138.295999 90.495999) (end 138.3 90.5) (width 0.254) (layer B.Cu) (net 10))
 (segment (start 138.295999 88.304001) (end 138.295999 90.495999) (width 0.254) (layer B.Cu) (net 10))
 (segment (start 138.85 87.75) (end 138.295999 88.304001) (width 0.254) (layer B.Cu) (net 10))
 (segment (start 138.3 90.5) (end 138.9 91.1) (width 0.254) (layer F.Cu) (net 10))
 (via (at 137 95.6) (size 0.6) (drill 0.4) (layers F.Cu B.Cu) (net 10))
 (segment (start 137 95.6) (end 137 94.4) (width 0.254) (layer B.Cu) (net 10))
 (via (at 133.026461 97.973539) (size 0.6) (drill 0.4) (layers F.Cu B.Cu) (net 10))
 (segment (start 135.4 95.6) (end 133.026461 97.973539) (width 0.254) (layer F.Cu) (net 10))
 (segment (start 137 95.6) (end 135.4 95.6) (width 0.254) (layer F.Cu) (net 10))
 (segment (start 133.026461 98.676461) (end 133.35 99) (width 0.254) (layer B.Cu) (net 10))
 (segment (start 133.026461 97.973539) (end 133.026461 98.676461) (width 0.254) (layer B.Cu) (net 10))
 (segment (start 137 95.6) (end 138.4 95.6) (width 0.254) (layer F.Cu) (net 10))
 (segment (start 138.4 95.6) (end 139.3 94.7) (width 0.254) (layer F.Cu) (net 10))
 (segment (start 139.3 91.5) (end 138.9 91.1) (width 0.254) (layer F.Cu) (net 10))
 (segment (start 139.3 94.7) (end 139.3 91.5) (width 0.254) (layer F.Cu) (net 10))
 (segment (start 137.7625 93.175) (end 139.525 93.175) (width 0.2) (layer B.Cu) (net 11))
 (via (at 140.454 92.5) (size 0.6) (drill 0.4) (layers F.Cu B.Cu) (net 11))
 (segment (start 139.779 93.175) (end 140.454 92.5) (width 0.254) (layer B.Cu) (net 11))
 (segment (start 139.525 93.175) (end 139.779 93.175) (width 0.254) (layer B.Cu) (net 11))
 (via (at 140 88.5) (size 0.6) (drill 0.4) (layers F.Cu B.Cu) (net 11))
 (segment (start 140.454 88.954) (end 140 88.5) (width 0.254) (layer F.Cu) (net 11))
 (segment (start 140.454 92.5) (end 140.454 88.954) (width 0.254) (layer F.Cu) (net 11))
 (segment (start 140.25 88.5) (end 141 87.75) (width 0.254) (layer B.Cu) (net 11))
 (segment (start 140 88.5) (end 140.25 88.5) (width 0.254) (layer B.Cu) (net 11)))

